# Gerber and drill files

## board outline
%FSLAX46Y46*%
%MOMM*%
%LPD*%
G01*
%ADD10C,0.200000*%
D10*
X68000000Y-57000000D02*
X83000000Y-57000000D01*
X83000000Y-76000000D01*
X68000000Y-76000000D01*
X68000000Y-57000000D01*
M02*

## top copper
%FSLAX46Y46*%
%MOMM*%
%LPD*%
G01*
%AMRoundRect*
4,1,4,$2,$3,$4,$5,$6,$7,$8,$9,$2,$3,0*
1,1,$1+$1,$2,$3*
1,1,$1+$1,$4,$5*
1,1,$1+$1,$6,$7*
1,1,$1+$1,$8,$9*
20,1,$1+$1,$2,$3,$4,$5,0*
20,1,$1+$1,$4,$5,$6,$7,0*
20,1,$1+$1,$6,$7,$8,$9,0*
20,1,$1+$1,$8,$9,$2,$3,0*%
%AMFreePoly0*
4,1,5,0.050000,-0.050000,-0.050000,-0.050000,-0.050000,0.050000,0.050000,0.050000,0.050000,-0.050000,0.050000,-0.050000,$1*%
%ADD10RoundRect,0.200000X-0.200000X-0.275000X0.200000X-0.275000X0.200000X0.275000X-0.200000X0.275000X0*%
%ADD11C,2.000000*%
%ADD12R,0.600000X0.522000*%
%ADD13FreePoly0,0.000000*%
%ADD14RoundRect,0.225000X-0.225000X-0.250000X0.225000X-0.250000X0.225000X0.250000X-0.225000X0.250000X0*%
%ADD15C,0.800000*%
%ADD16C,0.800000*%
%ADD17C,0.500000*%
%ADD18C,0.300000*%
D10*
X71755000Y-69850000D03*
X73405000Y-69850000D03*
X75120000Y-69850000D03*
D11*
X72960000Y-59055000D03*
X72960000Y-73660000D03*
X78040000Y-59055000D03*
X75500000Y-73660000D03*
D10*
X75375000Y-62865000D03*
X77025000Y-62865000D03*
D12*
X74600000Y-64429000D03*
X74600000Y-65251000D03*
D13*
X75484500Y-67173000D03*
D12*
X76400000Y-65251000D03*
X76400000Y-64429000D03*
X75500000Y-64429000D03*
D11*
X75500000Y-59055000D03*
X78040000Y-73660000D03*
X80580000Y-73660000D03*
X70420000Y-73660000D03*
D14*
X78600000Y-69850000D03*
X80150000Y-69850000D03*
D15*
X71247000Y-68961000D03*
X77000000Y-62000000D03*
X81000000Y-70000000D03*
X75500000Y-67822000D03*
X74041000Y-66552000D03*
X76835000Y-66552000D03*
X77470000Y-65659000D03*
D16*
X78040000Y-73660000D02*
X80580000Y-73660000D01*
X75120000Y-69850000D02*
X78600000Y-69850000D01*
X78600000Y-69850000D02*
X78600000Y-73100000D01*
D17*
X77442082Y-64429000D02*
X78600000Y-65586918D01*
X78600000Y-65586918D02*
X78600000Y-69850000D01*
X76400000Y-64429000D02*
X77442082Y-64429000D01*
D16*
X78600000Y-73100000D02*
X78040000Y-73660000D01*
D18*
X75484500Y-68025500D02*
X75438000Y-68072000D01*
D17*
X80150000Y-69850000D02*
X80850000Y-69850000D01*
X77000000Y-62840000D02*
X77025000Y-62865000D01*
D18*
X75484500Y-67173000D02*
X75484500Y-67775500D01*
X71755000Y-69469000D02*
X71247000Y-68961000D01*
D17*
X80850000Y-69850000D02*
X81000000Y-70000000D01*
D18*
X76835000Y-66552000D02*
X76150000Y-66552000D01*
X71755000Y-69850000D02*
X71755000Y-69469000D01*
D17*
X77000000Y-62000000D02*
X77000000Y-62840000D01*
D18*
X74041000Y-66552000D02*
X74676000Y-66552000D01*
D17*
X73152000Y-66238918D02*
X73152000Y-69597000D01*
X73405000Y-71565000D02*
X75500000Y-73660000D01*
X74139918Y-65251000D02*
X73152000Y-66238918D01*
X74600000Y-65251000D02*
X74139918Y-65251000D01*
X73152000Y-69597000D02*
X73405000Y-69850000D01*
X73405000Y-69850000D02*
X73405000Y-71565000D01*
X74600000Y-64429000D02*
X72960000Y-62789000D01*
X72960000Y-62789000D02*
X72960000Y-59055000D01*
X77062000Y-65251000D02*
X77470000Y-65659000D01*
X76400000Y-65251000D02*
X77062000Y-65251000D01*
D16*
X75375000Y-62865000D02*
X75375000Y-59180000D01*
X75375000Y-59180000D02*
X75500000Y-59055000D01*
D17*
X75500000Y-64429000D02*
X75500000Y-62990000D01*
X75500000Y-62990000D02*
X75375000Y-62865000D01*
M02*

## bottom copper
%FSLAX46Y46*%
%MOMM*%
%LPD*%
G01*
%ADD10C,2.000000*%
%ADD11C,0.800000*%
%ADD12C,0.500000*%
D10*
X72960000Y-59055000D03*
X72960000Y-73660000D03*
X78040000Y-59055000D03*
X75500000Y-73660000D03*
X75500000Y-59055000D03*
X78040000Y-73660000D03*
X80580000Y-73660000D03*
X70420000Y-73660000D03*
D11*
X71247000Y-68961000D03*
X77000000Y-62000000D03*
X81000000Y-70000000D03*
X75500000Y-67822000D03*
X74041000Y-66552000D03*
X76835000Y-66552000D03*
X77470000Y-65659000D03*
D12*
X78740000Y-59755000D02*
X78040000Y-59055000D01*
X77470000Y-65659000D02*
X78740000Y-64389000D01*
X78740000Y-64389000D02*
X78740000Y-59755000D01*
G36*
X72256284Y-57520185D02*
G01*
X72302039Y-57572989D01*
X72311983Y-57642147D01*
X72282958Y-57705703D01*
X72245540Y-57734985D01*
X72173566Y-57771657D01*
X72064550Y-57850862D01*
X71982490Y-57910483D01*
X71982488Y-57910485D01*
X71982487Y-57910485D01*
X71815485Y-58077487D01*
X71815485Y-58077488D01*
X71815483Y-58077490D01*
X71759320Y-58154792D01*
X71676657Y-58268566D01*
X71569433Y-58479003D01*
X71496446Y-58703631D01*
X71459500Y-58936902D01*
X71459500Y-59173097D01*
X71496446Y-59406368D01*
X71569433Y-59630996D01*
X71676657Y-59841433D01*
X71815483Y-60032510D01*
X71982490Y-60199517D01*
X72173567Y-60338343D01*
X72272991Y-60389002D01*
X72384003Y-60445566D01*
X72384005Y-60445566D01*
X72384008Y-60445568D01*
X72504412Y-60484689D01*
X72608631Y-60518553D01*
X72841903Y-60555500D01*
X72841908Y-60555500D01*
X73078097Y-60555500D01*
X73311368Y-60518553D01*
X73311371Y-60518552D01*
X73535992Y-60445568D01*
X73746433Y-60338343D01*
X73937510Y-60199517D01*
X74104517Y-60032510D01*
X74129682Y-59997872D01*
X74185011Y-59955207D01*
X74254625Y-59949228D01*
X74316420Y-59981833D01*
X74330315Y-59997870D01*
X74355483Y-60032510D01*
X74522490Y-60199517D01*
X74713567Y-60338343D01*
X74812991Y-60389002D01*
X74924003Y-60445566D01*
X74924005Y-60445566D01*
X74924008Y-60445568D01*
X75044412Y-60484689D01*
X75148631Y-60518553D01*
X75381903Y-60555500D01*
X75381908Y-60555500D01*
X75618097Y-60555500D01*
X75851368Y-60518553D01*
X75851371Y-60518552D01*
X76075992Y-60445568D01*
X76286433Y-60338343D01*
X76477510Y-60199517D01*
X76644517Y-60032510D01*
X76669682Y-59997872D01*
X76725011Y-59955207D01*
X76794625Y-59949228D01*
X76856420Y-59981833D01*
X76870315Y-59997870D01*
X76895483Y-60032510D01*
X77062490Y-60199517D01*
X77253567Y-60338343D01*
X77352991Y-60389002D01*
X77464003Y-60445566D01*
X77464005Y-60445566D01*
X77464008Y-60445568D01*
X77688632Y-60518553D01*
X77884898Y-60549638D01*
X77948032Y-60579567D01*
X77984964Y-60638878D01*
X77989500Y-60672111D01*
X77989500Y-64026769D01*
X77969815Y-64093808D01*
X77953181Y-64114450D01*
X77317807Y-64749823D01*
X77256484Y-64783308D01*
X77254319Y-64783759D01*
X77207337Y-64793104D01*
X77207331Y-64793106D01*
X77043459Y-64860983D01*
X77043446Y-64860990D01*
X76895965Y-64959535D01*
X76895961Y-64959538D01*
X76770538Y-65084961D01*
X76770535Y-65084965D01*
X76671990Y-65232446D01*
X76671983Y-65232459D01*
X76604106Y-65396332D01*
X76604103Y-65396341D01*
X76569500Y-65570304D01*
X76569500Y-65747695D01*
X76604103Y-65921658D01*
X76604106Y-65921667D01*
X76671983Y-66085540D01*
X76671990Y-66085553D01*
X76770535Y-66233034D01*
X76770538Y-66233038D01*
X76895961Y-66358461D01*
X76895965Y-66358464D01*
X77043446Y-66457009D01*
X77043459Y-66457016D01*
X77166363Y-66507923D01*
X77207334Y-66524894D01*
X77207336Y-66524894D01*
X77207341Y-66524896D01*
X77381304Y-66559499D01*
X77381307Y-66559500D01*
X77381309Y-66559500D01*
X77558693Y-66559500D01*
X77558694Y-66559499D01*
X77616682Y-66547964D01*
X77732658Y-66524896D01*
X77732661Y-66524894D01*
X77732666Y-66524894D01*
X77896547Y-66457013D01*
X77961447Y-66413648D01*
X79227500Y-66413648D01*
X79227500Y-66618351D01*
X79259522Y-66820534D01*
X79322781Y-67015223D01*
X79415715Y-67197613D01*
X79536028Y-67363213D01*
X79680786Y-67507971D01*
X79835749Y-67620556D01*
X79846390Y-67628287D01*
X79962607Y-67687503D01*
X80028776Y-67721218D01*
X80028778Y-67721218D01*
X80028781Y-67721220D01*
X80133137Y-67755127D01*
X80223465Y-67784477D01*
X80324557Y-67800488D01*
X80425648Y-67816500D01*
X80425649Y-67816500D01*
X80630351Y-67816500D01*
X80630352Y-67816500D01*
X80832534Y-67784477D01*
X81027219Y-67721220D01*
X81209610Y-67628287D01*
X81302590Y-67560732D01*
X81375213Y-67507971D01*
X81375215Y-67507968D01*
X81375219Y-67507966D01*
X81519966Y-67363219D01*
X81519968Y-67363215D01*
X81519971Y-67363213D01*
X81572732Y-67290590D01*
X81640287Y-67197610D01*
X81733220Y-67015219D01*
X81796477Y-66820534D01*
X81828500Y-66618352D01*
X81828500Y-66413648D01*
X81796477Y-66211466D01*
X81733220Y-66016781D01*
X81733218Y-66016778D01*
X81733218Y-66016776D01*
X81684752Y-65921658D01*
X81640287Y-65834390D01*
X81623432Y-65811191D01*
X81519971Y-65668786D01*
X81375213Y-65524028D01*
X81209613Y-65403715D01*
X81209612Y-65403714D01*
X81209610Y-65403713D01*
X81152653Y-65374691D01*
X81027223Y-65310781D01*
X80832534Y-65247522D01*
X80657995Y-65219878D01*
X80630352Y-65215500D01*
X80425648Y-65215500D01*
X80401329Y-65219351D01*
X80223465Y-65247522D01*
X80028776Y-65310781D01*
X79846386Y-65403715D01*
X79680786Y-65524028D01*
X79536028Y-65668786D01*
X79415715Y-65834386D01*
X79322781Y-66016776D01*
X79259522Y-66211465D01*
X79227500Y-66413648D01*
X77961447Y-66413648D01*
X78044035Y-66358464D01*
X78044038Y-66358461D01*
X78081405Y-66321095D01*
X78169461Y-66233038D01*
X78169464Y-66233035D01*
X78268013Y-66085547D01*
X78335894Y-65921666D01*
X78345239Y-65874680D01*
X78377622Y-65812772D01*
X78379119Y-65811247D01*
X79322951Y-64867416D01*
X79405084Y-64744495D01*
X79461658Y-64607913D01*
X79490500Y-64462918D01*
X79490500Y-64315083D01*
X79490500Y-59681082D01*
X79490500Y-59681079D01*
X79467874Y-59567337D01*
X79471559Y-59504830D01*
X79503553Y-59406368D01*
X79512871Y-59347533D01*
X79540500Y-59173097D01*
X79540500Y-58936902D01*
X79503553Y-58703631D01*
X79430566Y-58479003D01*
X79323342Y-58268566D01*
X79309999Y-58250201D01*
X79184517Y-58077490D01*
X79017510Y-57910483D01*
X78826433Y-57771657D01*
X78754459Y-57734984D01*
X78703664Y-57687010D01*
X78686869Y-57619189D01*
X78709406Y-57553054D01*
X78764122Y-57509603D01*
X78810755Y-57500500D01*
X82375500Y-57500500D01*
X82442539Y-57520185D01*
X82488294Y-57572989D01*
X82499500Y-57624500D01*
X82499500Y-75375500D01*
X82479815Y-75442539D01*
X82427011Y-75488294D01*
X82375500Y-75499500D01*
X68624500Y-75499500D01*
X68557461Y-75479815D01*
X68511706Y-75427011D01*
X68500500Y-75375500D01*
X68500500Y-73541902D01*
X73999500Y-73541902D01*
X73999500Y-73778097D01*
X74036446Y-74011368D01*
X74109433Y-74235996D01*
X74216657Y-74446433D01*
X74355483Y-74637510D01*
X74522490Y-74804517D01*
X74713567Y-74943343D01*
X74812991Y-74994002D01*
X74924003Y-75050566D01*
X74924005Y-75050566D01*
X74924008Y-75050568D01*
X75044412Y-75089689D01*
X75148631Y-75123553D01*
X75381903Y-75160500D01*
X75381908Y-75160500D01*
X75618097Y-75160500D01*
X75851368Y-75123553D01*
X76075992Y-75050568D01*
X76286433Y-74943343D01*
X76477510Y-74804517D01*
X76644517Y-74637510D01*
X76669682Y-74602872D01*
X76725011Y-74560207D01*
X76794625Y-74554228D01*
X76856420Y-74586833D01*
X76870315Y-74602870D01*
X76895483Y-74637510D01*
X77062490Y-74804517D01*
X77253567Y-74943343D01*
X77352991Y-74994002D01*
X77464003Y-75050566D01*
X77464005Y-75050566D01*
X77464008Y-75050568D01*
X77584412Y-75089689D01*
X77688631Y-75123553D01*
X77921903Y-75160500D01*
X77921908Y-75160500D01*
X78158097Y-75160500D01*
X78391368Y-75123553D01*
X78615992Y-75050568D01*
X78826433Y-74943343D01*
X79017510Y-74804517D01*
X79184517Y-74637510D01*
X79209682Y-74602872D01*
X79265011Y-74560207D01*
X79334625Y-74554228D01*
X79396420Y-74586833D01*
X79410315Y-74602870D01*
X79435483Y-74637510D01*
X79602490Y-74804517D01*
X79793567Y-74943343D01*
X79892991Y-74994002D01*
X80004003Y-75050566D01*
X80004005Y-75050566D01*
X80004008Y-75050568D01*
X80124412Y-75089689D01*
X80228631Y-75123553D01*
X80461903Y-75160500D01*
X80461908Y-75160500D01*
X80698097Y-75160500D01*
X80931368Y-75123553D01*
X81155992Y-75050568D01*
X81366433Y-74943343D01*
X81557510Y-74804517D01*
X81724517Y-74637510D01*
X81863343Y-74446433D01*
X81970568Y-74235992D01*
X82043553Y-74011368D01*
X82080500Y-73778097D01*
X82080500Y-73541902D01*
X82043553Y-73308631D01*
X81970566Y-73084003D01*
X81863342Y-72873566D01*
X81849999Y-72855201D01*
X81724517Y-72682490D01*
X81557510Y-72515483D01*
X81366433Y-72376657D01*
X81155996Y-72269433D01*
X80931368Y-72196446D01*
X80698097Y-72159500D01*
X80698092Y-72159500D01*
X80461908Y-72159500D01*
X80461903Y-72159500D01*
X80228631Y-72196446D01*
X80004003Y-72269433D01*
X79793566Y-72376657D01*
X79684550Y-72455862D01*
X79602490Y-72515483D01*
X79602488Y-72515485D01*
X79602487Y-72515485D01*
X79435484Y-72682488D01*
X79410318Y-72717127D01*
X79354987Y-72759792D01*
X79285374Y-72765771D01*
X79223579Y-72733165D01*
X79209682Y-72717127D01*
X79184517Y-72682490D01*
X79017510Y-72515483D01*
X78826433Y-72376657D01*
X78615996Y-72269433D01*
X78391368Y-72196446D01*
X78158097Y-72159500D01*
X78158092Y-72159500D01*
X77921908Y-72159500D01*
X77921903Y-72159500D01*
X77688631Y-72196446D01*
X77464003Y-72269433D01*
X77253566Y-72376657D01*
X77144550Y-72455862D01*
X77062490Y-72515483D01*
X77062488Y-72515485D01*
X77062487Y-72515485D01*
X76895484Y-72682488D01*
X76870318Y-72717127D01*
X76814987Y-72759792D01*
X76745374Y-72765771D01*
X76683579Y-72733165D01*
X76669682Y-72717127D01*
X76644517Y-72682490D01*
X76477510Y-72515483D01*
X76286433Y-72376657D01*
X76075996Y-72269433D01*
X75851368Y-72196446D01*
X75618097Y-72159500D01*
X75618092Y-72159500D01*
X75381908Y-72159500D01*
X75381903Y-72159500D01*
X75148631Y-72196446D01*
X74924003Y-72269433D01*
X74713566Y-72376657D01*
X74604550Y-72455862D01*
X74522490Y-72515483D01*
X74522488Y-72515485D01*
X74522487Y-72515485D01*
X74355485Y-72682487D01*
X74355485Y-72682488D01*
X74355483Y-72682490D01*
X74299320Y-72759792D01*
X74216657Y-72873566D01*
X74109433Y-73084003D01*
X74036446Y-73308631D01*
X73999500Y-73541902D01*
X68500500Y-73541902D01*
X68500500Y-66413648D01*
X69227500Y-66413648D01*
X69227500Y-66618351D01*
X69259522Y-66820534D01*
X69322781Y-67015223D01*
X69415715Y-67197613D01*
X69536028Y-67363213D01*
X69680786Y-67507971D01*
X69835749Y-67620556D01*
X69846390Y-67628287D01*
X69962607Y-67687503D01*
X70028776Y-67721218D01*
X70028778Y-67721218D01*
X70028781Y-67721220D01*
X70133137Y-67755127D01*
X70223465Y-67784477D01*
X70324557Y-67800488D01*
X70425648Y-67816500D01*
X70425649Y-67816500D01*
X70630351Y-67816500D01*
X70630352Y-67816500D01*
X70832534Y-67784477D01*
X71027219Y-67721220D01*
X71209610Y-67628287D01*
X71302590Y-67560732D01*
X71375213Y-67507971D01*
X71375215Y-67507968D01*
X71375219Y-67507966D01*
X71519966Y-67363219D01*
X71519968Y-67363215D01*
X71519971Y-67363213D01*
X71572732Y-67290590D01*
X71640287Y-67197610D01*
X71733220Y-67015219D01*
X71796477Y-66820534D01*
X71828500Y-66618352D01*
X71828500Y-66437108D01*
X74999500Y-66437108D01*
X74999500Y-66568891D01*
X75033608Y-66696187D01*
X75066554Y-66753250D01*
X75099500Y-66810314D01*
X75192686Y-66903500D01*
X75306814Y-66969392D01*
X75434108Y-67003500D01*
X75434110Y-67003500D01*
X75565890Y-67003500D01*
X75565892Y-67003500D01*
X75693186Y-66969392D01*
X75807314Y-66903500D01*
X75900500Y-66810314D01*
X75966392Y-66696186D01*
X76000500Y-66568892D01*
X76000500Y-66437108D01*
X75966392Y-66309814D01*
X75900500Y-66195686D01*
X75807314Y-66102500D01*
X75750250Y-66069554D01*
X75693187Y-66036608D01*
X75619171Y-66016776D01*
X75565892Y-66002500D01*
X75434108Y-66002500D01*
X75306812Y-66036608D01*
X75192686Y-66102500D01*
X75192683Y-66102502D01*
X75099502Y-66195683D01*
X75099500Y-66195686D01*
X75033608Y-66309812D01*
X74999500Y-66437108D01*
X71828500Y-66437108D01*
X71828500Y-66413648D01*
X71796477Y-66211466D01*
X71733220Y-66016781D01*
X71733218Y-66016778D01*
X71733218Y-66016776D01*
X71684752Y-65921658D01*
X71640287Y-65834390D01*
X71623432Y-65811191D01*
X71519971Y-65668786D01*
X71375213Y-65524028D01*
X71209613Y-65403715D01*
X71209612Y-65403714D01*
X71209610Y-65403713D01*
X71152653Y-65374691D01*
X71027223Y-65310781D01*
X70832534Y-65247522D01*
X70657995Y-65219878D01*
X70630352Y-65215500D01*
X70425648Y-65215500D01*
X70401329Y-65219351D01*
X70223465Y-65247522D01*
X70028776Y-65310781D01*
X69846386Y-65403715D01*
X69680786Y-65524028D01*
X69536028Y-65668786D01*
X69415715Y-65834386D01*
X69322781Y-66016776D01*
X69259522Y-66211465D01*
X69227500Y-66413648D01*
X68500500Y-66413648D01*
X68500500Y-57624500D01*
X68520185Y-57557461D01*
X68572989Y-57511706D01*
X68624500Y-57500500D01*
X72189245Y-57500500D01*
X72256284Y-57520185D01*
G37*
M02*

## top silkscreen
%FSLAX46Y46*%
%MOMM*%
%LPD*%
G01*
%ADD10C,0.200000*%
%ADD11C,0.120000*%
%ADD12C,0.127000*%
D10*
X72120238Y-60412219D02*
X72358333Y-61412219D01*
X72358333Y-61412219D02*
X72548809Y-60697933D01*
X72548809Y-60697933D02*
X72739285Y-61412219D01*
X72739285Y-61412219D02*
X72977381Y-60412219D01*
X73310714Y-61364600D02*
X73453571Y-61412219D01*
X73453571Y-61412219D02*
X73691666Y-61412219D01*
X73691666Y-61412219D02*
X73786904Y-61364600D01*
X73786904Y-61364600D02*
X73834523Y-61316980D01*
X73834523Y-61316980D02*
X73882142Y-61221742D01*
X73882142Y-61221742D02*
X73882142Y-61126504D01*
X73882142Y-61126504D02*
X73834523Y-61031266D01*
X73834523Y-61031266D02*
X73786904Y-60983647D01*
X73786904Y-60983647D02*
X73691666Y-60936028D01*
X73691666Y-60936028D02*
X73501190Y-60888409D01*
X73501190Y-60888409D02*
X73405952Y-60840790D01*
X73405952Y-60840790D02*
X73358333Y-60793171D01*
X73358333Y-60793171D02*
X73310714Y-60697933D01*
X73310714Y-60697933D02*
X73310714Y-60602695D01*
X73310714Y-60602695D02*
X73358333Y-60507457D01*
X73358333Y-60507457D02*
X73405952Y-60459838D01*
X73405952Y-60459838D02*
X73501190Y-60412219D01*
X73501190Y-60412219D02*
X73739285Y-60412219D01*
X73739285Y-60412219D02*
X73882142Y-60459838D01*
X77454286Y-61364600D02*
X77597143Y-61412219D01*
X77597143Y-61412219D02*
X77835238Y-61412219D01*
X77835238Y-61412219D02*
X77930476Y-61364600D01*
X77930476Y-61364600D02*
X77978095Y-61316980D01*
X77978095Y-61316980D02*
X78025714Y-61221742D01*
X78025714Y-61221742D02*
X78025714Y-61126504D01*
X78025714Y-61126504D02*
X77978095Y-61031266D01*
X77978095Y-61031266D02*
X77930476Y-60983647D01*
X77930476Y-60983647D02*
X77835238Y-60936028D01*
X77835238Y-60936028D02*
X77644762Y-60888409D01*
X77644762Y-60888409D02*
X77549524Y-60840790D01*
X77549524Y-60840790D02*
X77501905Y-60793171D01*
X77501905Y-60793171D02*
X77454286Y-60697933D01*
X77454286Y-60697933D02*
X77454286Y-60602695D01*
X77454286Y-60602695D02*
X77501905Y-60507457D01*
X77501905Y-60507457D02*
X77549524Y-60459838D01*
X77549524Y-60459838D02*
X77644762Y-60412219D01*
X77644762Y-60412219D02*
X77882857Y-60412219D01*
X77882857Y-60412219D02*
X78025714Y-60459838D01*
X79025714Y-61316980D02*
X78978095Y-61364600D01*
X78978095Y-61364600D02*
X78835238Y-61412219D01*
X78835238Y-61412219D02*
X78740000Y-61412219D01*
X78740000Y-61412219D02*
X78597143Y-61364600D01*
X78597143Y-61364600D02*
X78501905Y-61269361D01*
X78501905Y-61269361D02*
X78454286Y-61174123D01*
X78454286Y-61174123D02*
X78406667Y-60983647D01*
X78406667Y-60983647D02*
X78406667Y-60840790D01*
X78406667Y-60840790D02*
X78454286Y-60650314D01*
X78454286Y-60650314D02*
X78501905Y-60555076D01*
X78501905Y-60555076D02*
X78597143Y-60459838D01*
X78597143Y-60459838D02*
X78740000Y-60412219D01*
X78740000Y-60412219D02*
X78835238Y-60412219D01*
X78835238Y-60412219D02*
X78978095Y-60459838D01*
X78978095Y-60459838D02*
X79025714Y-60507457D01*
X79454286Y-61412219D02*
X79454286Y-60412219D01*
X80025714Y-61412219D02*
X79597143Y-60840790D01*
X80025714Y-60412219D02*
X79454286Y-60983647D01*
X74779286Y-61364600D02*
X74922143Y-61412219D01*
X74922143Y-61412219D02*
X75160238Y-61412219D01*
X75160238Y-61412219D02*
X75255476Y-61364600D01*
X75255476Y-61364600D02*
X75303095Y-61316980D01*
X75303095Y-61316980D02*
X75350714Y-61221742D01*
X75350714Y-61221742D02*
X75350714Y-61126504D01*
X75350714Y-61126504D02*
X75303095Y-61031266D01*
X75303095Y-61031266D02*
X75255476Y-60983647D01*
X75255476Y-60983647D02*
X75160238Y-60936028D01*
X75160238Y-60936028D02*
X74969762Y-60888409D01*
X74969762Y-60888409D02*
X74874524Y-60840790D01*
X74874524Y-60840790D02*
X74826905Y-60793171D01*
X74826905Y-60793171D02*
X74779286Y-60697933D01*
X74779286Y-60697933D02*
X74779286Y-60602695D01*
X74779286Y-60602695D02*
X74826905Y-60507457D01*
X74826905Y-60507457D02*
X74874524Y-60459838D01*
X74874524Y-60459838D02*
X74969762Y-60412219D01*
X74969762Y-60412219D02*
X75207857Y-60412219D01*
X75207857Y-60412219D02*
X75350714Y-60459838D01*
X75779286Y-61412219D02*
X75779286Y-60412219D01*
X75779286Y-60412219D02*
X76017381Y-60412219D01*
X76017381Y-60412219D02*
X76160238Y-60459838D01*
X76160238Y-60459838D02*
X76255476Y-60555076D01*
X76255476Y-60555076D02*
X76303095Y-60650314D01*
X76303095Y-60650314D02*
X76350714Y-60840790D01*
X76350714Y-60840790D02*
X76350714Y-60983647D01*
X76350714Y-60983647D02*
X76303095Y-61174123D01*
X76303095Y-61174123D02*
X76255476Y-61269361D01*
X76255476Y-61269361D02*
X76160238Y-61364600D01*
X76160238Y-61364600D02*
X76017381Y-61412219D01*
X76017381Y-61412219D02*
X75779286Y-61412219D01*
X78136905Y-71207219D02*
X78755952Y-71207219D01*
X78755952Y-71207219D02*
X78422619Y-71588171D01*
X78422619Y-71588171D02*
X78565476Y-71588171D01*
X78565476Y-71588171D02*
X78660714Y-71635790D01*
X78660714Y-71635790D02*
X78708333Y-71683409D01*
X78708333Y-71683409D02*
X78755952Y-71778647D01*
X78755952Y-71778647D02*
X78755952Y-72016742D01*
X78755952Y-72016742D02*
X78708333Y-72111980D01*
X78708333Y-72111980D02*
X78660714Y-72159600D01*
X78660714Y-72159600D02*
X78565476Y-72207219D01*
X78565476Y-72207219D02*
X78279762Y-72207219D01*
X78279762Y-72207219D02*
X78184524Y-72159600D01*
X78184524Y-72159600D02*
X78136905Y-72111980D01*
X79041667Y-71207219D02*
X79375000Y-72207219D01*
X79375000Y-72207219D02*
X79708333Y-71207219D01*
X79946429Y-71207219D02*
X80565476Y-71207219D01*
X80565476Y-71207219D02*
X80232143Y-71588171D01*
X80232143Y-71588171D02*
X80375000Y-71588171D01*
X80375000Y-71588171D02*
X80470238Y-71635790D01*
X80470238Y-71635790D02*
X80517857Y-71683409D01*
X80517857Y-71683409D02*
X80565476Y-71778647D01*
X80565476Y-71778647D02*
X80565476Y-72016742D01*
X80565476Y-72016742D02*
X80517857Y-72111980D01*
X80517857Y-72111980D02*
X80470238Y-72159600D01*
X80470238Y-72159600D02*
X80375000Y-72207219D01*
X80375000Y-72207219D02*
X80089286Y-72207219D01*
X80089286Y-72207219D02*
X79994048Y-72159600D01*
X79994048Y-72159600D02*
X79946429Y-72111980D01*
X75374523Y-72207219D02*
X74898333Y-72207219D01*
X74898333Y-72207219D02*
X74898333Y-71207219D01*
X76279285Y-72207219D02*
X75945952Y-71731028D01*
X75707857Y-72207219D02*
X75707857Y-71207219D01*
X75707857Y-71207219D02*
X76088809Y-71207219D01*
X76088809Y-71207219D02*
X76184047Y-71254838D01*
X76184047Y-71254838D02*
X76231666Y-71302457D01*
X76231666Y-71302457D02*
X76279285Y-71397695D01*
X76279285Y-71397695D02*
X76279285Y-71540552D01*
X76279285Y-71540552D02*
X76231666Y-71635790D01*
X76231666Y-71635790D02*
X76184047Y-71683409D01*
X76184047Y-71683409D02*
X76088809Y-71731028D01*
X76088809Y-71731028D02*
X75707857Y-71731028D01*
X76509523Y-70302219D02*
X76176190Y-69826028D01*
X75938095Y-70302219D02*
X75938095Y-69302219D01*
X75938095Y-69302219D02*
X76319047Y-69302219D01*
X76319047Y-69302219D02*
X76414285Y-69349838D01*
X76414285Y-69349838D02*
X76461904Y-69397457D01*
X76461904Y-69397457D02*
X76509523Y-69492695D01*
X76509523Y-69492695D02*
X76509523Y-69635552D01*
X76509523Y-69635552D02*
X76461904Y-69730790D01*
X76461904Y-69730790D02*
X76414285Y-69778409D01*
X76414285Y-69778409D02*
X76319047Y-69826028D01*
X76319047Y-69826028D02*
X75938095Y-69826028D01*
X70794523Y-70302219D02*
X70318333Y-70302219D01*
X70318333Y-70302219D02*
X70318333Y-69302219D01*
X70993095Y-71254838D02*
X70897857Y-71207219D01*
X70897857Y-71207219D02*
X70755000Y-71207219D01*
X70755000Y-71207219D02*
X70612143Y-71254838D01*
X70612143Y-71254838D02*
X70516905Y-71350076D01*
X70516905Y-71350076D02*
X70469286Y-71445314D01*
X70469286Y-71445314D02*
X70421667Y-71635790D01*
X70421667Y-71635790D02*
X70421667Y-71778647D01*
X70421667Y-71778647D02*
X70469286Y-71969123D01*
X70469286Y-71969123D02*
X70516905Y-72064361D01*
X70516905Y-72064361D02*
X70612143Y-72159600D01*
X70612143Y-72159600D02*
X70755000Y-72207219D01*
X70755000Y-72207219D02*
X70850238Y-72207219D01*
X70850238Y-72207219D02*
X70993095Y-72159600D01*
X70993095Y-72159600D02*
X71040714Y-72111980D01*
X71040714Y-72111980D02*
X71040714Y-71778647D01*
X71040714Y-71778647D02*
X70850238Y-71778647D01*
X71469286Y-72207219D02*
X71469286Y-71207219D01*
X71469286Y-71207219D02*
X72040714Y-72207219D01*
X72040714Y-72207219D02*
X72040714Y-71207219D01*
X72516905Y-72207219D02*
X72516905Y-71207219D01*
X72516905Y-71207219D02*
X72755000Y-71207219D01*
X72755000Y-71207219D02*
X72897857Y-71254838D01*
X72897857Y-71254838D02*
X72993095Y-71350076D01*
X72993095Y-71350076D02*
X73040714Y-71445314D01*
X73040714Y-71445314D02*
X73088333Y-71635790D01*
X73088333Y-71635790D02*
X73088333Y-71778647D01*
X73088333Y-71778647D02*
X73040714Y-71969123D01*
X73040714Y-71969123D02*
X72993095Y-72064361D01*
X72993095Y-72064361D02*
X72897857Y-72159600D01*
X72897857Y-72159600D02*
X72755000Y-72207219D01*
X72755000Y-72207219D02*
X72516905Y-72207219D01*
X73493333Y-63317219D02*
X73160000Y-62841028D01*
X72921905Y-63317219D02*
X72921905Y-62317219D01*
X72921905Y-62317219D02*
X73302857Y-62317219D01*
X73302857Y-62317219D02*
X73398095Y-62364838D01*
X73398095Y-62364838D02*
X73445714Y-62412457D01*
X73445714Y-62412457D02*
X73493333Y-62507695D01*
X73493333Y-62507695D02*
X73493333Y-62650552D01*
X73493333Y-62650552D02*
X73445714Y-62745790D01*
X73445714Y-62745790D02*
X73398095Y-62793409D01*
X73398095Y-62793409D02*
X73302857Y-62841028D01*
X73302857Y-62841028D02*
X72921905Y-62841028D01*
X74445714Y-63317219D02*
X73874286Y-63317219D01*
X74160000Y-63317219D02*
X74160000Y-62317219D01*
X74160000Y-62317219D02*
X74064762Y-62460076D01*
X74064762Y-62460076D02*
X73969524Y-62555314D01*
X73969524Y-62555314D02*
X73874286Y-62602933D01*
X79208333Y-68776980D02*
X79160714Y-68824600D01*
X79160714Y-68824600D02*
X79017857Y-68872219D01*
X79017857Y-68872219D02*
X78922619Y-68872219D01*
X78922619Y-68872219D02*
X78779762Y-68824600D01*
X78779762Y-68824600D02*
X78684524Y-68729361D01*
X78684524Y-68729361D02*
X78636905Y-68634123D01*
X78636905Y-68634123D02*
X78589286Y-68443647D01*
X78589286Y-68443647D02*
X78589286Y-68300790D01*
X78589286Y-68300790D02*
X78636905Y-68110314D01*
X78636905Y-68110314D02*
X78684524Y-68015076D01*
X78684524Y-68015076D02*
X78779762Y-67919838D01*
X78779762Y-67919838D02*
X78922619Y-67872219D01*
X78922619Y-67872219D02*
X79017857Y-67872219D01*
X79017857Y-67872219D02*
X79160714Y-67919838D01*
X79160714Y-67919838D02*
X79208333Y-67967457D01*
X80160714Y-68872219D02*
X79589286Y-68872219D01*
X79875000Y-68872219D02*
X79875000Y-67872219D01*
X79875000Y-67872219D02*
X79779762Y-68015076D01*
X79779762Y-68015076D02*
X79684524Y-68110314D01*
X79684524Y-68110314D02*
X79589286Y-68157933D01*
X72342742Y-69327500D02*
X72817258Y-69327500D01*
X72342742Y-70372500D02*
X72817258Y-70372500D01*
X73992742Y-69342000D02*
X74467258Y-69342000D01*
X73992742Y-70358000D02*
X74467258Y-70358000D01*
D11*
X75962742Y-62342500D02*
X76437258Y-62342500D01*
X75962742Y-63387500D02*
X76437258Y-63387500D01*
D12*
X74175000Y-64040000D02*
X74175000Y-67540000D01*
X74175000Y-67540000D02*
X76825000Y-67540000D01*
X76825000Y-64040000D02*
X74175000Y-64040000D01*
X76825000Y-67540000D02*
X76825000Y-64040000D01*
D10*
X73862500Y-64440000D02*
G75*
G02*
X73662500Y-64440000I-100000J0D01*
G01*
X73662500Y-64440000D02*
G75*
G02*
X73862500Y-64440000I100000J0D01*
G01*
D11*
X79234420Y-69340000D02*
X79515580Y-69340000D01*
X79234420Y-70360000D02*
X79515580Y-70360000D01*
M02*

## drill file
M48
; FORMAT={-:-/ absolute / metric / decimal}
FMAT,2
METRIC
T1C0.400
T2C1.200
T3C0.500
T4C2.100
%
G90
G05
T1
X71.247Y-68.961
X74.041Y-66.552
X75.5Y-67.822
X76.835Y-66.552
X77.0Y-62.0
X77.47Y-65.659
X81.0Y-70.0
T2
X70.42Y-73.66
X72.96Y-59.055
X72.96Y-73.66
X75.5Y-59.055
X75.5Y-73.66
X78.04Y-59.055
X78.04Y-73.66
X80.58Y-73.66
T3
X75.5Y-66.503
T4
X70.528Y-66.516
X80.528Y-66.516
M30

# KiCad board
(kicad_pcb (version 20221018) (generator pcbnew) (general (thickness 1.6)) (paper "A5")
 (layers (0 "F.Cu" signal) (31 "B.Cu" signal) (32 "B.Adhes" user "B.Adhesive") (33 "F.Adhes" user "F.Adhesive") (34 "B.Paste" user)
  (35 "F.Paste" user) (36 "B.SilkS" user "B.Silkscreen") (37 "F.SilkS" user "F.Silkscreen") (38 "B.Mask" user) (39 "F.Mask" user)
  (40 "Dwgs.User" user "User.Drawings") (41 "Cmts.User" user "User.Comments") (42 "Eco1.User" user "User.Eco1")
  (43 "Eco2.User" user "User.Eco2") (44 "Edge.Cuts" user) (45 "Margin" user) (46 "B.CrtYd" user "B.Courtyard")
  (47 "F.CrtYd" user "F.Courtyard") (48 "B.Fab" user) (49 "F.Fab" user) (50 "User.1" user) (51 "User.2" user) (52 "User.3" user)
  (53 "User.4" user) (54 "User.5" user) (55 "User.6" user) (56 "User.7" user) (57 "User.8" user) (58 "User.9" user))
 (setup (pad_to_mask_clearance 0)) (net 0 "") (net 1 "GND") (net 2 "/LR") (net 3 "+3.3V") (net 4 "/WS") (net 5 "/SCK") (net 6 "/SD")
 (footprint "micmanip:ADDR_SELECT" (layer "F.Cu") (at 73.43 69.8375)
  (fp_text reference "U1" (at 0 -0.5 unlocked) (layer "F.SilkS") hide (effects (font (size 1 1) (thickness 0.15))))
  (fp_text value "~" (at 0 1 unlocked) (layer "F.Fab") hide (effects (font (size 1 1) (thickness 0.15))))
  (fp_line (start -1.087258 -0.51) (end -0.612742 -0.51) (stroke (width 0.2) (type solid)) (layer "F.SilkS"))
  (fp_line (start -1.087258 0.535) (end -0.612742 0.535) (stroke (width 0.2) (type solid)) (layer "F.SilkS"))
  (fp_line (start 0.562742 -0.4955) (end 1.037258 -0.4955) (stroke (width 0.2) (type solid)) (layer "F.SilkS"))
  (fp_line (start 0.562742 0.5205) (end 1.037258 0.5205) (stroke (width 0.2) (type solid)) (layer "F.SilkS"))
  (pad "1" smd roundrect (at -1.675 0.0125) (size 0.8 0.95) (layers "F.Cu" "F.Paste" "F.Mask") (roundrect_rratio 0.25) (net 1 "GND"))
  (pad "2" smd roundrect (at -0.025 0.0125) (size 0.8 0.95) (layers "F.Cu" "F.Paste" "F.Mask") (roundrect_rratio 0.25) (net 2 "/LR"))
  (pad "3" smd roundrect (at 1.69 0.0125) (size 0.8 0.95) (layers "F.Cu" "F.Paste" "F.Mask") (roundrect_rratio 0.25) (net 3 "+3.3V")))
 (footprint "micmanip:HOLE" (layer "F.Cu") (at 72.96 59.055)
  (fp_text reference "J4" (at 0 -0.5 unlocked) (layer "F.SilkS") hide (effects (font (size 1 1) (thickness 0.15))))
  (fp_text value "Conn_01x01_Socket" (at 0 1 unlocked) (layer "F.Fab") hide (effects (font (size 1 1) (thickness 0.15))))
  (pad "1" thru_hole circle (at 0 0) (size 2 2) (drill 1.2) (layers "*.Cu" "*.Mask") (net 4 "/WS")))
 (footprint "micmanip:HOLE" (layer "F.Cu") (at 72.96 73.66)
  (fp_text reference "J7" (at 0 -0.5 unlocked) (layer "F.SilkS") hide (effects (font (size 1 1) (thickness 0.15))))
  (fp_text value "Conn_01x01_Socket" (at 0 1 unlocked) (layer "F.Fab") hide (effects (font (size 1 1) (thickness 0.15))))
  (pad "1" thru_hole circle (at 0 0) (size 2 2) (drill 1.2) (layers "*.Cu" "*.Mask") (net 1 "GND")))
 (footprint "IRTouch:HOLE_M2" (layer "F.Cu") (at 80.5 66.5)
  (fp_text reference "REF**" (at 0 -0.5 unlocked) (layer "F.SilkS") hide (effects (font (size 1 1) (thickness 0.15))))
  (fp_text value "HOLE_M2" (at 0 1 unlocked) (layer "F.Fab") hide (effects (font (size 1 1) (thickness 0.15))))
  (pad "" np_thru_hole circle (at 0.028 0.016) (size 1.5 1.5) (drill 2.1) (layers "F&B.Cu" "*.Mask")))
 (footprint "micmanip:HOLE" (layer "F.Cu") (at 78.04 59.055)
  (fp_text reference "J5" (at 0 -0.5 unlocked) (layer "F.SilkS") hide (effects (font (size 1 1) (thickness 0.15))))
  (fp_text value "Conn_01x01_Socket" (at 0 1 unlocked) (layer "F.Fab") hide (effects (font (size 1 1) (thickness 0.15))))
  (pad "1" thru_hole circle (at 0 0) (size 2 2) (drill 1.2) (layers "*.Cu" "*.Mask") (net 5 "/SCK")))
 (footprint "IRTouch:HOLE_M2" (layer "F.Cu") (at 70.5 66.5)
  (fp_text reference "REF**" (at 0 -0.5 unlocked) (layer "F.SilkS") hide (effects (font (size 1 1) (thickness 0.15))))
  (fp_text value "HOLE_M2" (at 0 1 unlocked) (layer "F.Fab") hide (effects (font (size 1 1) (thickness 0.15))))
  (pad "" np_thru_hole circle (at 0.028 0.016) (size 1.5 1.5) (drill 2.1) (layers "F&B.Cu" "*.Mask")))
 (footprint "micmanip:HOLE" (layer "F.Cu") (at 75.5 73.66)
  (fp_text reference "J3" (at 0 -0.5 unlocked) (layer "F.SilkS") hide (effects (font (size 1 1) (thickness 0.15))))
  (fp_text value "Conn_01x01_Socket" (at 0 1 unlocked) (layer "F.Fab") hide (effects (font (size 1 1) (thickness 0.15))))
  (pad "1" thru_hole circle (at 0 0) (size 2 2) (drill 1.2) (layers "*.Cu" "*.Mask") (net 2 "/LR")))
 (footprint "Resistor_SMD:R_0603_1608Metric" (layer "F.Cu") (at 76.2 62.865)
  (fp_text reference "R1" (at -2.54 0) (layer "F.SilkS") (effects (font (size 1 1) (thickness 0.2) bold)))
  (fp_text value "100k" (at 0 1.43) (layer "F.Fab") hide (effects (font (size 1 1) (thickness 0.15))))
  (fp_line (start -0.237258 -0.5225) (end 0.237258 -0.5225) (stroke (width 0.12) (type solid)) (layer "F.SilkS"))
  (fp_line (start -0.237258 0.5225) (end 0.237258 0.5225) (stroke (width 0.12) (type solid)) (layer "F.SilkS"))
  (pad "1" smd roundrect (at -0.825 0) (size 0.8 0.95) (layers "F.Cu" "F.Paste" "F.Mask") (roundrect_rratio 0.25) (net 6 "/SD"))
  (pad "2" smd roundrect (at 0.825 0) (size 0.8 0.95) (layers "F.Cu" "F.Paste" "F.Mask") (roundrect_rratio 0.25) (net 1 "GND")))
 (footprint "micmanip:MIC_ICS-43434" (layer "F.Cu") (at 75.5 65.79)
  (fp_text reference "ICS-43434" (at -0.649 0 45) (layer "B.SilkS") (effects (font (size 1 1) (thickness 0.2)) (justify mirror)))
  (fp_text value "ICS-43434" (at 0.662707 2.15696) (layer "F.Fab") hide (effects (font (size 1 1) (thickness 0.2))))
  (fp_line (start -1.325 -1.75) (end -1.325 1.75) (stroke (width 0.127) (type solid)) (layer "F.SilkS"))
  (fp_line (start -1.325 1.75) (end 1.325 1.75) (stroke (width 0.127) (type solid)) (layer "F.SilkS"))
  (fp_line (start 1.325 -1.75) (end -1.325 -1.75) (stroke (width 0.127) (type solid)) (layer "F.SilkS"))
  (fp_line (start 1.325 1.75) (end 1.325 -1.75) (stroke (width 0.127) (type solid)) (layer "F.SilkS"))
  (fp_circle (center -1.7375 -1.35) (end -1.6375 -1.35) (stroke (width 0.2) (type solid)) (fill none) (layer "F.SilkS"))
  (pad "" np_thru_hole circle (at 0 0.713) (size 0.5 0.5) (drill 0.5) (layers "*.Cu" "*.Mask"))
  (pad "1" smd rect (at -0.9 -1.361) (size 0.6 0.522) (layers "F.Cu" "F.Mask") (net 4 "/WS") (solder_mask_margin 0.102))
  (pad "2" smd rect (at -0.9 -0.539) (size 0.6 0.522) (layers "F.Cu" "F.Mask") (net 2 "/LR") (solder_mask_margin 0.102))
  (pad "3" smd custom (at -0.0155 1.383) (size 0.1 0.1) (layers "F.Cu") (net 1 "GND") (thermal_bridge_angle 45)
   (options (clearance outline) (anchor rect)) (primitives))
  (pad "4" smd rect (at 0.9 -0.539) (size 0.6 0.522) (layers "F.Cu" "F.Mask") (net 5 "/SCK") (solder_mask_margin 0.102))
  (pad "5" smd rect (at 0.9 -1.361) (size 0.6 0.522) (layers "F.Cu" "F.Mask") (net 3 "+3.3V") (solder_mask_margin 0.102))
  (pad "6" smd rect (at 0 -1.361) (size 0.6 0.522) (layers "F.Cu" "F.Mask") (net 6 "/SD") (solder_mask_margin 0.102)))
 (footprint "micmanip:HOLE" (layer "F.Cu") (at 75.5 59.055)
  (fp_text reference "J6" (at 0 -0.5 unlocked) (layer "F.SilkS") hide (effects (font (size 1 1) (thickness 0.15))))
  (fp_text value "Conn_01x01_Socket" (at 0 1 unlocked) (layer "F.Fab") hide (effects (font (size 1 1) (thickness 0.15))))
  (pad "1" thru_hole circle (at 0 0) (size 2 2) (drill 1.2) (layers "*.Cu" "*.Mask") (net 6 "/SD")))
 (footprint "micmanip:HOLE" (layer "F.Cu") (at 78.04 73.66)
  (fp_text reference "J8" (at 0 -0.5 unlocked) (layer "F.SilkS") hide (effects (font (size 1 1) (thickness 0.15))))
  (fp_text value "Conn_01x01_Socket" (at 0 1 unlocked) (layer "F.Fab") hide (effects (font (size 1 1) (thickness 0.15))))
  (pad "1" thru_hole circle (at 0 0) (size 2 2) (drill 1.2) (layers "*.Cu" "*.Mask") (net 3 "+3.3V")))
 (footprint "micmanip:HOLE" (layer "F.Cu") (at 80.58 73.66)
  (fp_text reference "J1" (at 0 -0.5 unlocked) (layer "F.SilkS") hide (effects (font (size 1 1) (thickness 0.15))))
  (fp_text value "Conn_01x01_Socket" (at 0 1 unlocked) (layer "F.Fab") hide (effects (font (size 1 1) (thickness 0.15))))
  (pad "1" thru_hole circle (at 0 0) (size 2 2) (drill 1.2) (layers "*.Cu" "*.Mask") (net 3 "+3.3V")))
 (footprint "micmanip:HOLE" (layer "F.Cu") (at 70.42 73.66)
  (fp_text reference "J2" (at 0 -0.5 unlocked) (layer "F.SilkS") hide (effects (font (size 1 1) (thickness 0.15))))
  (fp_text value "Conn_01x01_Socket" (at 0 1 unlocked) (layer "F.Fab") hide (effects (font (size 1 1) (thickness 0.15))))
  (pad "1" thru_hole circle (at 0 0) (size 2 2) (drill 1.2) (layers "*.Cu" "*.Mask") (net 1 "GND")))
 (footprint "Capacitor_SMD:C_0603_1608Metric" (layer "F.Cu") (at 79.375 69.85)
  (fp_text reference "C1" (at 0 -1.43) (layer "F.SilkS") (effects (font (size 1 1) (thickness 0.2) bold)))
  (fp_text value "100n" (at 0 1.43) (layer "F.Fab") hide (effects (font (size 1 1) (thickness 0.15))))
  (fp_line (start -0.14058 -0.51) (end 0.14058 -0.51) (stroke (width 0.12) (type solid)) (layer "F.SilkS"))
  (fp_line (start -0.14058 0.51) (end 0.14058 0.51) (stroke (width 0.12) (type solid)) (layer "F.SilkS"))
  (pad "1" smd roundrect (at -0.775 0) (size 0.9 0.95) (layers "F.Cu" "F.Paste" "F.Mask") (roundrect_rratio 0.25) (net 3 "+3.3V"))
  (pad "2" smd roundrect (at 0.775 0) (size 0.9 0.95) (layers "F.Cu" "F.Paste" "F.Mask") (roundrect_rratio 0.25) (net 1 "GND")))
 (gr_rect (start 68 57) (end 83 76) (stroke (width 0.2) (type default)) (fill none) (layer "Edge.Cuts"))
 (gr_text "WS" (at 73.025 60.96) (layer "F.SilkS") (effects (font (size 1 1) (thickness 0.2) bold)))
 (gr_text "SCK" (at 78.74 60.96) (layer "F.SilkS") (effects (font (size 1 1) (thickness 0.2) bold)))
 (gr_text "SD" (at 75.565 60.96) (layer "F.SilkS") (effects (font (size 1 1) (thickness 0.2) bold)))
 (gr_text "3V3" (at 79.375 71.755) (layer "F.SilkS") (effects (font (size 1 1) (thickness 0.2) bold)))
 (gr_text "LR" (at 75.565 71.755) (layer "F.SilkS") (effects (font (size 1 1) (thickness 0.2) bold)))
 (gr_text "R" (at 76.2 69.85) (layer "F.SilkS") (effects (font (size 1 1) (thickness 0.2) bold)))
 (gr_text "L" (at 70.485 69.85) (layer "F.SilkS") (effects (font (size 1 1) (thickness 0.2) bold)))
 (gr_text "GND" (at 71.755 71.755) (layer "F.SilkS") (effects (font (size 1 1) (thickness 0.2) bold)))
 (segment (start 78.04 73.66) (end 80.58 73.66) (width 0.8) (layer "F.Cu") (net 3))
 (segment (start 75.12 69.85) (end 78.6 69.85) (width 0.8) (layer "F.Cu") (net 3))
 (segment (start 78.6 69.85) (end 78.6 73.1) (width 0.8) (layer "F.Cu") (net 3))
 (segment (start 77.442082 64.429) (end 78.6 65.586918) (width 0.5) (layer "F.Cu") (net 3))
 (segment (start 78.6 65.586918) (end 78.6 69.85) (width 0.5) (layer "F.Cu") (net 3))
 (segment (start 76.4 64.429) (end 77.442082 64.429) (width 0.5) (layer "F.Cu") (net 3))
 (segment (start 78.6 73.1) (end 78.04 73.66) (width 0.8) (layer "F.Cu") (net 3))
 (segment (start 75.4845 68.0255) (end 75.438 68.072) (width 0.3) (layer "F.Cu") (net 1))
 (segment (start 80.15 69.85) (end 80.85 69.85) (width 0.5) (layer "F.Cu") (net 1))
 (segment (start 77 62.84) (end 77.025 62.865) (width 0.5) (layer "F.Cu") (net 1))
 (segment (start 75.4845 67.173) (end 75.4845 67.7755) (width 0.3) (layer "F.Cu") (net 1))
 (segment (start 71.755 69.469) (end 71.247 68.961) (width 0.3) (layer "F.Cu") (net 1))
 (segment (start 80.85 69.85) (end 81 70) (width 0.5) (layer "F.Cu") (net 1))
 (segment (start 76.835 66.552) (end 76.15 66.552) (width 0.3) (layer "F.Cu") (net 1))
 (segment (start 71.755 69.85) (end 71.755 69.469) (width 0.3) (layer "F.Cu") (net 1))
 (segment (start 77 62) (end 77 62.84) (width 0.5) (layer "F.Cu") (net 1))
 (segment (start 74.041 66.552) (end 74.676 66.552) (width 0.3) (layer "F.Cu") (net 1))
 (via (at 71.247 68.961) (size 0.8) (drill 0.4) (layers "F.Cu" "B.Cu") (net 1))
 (via (at 77 62) (size 0.8) (drill 0.4) (layers "F.Cu" "B.Cu") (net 1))
 (via (at 81 70) (size 0.8) (drill 0.4) (layers "F.Cu" "B.Cu") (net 1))
 (via (at 75.5 67.822) (size 0.8) (drill 0.4) (layers "F.Cu" "B.Cu") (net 1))
 (via (at 74.041 66.552) (size 0.8) (drill 0.4) (layers "F.Cu" "B.Cu") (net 1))
 (via (at 76.835 66.552) (size 0.8) (drill 0.4) (layers "F.Cu" "B.Cu") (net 1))
 (segment (start 73.152 66.238918) (end 73.152 69.597) (width 0.5) (layer "F.Cu") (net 2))
 (segment (start 73.405 71.565) (end 75.5 73.66) (width 0.5) (layer "F.Cu") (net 2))
 (segment (start 74.139918 65.251) (end 73.152 66.238918) (width 0.5) (layer "F.Cu") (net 2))
 (segment (start 74.6 65.251) (end 74.139918 65.251) (width 0.5) (layer "F.Cu") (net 2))
 (segment (start 73.152 69.597) (end 73.405 69.85) (width 0.5) (layer "F.Cu") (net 2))
 (segment (start 73.405 69.85) (end 73.405 71.565) (width 0.5) (layer "F.Cu") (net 2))
 (segment (start 74.6 64.429) (end 72.96 62.789) (width 0.5) (layer "F.Cu") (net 4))
 (segment (start 72.96 62.789) (end 72.96 59.055) (width 0.5) (layer "F.Cu") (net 4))
 (segment (start 77.062 65.251) (end 77.47 65.659) (width 0.5) (layer "F.Cu") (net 5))
 (segment (start 76.4 65.251) (end 77.062 65.251) (width 0.5) (layer "F.Cu") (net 5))
 (via (at 77.47 65.659) (size 0.8) (drill 0.4) (layers "F.Cu" "B.Cu") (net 5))
 (segment (start 78.74 59.755) (end 78.04 59.055) (width 0.5) (layer "B.Cu") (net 5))
 (segment (start 77.47 65.659) (end 78.74 64.389) (width 0.5) (layer "B.Cu") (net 5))
 (segment (start 78.74 64.389) (end 78.74 59.755) (width 0.5) (layer "B.Cu") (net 5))
 (segment (start 75.375 62.865) (end 75.375 59.18) (width 0.8) (layer "F.Cu") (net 6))
 (segment (start 75.375 59.18) (end 75.5 59.055) (width 0.8) (layer "F.Cu") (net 6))
 (segment (start 75.5 64.429) (end 75.5 62.99) (width 0.5) (layer "F.Cu") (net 6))
 (segment (start 75.5 62.99) (end 75.375 62.865) (width 0.5) (layer "F.Cu") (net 6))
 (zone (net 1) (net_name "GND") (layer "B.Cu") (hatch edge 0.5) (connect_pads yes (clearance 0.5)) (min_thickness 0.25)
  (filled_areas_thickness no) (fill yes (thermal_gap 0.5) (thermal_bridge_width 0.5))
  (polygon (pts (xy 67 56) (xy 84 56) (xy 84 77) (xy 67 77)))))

